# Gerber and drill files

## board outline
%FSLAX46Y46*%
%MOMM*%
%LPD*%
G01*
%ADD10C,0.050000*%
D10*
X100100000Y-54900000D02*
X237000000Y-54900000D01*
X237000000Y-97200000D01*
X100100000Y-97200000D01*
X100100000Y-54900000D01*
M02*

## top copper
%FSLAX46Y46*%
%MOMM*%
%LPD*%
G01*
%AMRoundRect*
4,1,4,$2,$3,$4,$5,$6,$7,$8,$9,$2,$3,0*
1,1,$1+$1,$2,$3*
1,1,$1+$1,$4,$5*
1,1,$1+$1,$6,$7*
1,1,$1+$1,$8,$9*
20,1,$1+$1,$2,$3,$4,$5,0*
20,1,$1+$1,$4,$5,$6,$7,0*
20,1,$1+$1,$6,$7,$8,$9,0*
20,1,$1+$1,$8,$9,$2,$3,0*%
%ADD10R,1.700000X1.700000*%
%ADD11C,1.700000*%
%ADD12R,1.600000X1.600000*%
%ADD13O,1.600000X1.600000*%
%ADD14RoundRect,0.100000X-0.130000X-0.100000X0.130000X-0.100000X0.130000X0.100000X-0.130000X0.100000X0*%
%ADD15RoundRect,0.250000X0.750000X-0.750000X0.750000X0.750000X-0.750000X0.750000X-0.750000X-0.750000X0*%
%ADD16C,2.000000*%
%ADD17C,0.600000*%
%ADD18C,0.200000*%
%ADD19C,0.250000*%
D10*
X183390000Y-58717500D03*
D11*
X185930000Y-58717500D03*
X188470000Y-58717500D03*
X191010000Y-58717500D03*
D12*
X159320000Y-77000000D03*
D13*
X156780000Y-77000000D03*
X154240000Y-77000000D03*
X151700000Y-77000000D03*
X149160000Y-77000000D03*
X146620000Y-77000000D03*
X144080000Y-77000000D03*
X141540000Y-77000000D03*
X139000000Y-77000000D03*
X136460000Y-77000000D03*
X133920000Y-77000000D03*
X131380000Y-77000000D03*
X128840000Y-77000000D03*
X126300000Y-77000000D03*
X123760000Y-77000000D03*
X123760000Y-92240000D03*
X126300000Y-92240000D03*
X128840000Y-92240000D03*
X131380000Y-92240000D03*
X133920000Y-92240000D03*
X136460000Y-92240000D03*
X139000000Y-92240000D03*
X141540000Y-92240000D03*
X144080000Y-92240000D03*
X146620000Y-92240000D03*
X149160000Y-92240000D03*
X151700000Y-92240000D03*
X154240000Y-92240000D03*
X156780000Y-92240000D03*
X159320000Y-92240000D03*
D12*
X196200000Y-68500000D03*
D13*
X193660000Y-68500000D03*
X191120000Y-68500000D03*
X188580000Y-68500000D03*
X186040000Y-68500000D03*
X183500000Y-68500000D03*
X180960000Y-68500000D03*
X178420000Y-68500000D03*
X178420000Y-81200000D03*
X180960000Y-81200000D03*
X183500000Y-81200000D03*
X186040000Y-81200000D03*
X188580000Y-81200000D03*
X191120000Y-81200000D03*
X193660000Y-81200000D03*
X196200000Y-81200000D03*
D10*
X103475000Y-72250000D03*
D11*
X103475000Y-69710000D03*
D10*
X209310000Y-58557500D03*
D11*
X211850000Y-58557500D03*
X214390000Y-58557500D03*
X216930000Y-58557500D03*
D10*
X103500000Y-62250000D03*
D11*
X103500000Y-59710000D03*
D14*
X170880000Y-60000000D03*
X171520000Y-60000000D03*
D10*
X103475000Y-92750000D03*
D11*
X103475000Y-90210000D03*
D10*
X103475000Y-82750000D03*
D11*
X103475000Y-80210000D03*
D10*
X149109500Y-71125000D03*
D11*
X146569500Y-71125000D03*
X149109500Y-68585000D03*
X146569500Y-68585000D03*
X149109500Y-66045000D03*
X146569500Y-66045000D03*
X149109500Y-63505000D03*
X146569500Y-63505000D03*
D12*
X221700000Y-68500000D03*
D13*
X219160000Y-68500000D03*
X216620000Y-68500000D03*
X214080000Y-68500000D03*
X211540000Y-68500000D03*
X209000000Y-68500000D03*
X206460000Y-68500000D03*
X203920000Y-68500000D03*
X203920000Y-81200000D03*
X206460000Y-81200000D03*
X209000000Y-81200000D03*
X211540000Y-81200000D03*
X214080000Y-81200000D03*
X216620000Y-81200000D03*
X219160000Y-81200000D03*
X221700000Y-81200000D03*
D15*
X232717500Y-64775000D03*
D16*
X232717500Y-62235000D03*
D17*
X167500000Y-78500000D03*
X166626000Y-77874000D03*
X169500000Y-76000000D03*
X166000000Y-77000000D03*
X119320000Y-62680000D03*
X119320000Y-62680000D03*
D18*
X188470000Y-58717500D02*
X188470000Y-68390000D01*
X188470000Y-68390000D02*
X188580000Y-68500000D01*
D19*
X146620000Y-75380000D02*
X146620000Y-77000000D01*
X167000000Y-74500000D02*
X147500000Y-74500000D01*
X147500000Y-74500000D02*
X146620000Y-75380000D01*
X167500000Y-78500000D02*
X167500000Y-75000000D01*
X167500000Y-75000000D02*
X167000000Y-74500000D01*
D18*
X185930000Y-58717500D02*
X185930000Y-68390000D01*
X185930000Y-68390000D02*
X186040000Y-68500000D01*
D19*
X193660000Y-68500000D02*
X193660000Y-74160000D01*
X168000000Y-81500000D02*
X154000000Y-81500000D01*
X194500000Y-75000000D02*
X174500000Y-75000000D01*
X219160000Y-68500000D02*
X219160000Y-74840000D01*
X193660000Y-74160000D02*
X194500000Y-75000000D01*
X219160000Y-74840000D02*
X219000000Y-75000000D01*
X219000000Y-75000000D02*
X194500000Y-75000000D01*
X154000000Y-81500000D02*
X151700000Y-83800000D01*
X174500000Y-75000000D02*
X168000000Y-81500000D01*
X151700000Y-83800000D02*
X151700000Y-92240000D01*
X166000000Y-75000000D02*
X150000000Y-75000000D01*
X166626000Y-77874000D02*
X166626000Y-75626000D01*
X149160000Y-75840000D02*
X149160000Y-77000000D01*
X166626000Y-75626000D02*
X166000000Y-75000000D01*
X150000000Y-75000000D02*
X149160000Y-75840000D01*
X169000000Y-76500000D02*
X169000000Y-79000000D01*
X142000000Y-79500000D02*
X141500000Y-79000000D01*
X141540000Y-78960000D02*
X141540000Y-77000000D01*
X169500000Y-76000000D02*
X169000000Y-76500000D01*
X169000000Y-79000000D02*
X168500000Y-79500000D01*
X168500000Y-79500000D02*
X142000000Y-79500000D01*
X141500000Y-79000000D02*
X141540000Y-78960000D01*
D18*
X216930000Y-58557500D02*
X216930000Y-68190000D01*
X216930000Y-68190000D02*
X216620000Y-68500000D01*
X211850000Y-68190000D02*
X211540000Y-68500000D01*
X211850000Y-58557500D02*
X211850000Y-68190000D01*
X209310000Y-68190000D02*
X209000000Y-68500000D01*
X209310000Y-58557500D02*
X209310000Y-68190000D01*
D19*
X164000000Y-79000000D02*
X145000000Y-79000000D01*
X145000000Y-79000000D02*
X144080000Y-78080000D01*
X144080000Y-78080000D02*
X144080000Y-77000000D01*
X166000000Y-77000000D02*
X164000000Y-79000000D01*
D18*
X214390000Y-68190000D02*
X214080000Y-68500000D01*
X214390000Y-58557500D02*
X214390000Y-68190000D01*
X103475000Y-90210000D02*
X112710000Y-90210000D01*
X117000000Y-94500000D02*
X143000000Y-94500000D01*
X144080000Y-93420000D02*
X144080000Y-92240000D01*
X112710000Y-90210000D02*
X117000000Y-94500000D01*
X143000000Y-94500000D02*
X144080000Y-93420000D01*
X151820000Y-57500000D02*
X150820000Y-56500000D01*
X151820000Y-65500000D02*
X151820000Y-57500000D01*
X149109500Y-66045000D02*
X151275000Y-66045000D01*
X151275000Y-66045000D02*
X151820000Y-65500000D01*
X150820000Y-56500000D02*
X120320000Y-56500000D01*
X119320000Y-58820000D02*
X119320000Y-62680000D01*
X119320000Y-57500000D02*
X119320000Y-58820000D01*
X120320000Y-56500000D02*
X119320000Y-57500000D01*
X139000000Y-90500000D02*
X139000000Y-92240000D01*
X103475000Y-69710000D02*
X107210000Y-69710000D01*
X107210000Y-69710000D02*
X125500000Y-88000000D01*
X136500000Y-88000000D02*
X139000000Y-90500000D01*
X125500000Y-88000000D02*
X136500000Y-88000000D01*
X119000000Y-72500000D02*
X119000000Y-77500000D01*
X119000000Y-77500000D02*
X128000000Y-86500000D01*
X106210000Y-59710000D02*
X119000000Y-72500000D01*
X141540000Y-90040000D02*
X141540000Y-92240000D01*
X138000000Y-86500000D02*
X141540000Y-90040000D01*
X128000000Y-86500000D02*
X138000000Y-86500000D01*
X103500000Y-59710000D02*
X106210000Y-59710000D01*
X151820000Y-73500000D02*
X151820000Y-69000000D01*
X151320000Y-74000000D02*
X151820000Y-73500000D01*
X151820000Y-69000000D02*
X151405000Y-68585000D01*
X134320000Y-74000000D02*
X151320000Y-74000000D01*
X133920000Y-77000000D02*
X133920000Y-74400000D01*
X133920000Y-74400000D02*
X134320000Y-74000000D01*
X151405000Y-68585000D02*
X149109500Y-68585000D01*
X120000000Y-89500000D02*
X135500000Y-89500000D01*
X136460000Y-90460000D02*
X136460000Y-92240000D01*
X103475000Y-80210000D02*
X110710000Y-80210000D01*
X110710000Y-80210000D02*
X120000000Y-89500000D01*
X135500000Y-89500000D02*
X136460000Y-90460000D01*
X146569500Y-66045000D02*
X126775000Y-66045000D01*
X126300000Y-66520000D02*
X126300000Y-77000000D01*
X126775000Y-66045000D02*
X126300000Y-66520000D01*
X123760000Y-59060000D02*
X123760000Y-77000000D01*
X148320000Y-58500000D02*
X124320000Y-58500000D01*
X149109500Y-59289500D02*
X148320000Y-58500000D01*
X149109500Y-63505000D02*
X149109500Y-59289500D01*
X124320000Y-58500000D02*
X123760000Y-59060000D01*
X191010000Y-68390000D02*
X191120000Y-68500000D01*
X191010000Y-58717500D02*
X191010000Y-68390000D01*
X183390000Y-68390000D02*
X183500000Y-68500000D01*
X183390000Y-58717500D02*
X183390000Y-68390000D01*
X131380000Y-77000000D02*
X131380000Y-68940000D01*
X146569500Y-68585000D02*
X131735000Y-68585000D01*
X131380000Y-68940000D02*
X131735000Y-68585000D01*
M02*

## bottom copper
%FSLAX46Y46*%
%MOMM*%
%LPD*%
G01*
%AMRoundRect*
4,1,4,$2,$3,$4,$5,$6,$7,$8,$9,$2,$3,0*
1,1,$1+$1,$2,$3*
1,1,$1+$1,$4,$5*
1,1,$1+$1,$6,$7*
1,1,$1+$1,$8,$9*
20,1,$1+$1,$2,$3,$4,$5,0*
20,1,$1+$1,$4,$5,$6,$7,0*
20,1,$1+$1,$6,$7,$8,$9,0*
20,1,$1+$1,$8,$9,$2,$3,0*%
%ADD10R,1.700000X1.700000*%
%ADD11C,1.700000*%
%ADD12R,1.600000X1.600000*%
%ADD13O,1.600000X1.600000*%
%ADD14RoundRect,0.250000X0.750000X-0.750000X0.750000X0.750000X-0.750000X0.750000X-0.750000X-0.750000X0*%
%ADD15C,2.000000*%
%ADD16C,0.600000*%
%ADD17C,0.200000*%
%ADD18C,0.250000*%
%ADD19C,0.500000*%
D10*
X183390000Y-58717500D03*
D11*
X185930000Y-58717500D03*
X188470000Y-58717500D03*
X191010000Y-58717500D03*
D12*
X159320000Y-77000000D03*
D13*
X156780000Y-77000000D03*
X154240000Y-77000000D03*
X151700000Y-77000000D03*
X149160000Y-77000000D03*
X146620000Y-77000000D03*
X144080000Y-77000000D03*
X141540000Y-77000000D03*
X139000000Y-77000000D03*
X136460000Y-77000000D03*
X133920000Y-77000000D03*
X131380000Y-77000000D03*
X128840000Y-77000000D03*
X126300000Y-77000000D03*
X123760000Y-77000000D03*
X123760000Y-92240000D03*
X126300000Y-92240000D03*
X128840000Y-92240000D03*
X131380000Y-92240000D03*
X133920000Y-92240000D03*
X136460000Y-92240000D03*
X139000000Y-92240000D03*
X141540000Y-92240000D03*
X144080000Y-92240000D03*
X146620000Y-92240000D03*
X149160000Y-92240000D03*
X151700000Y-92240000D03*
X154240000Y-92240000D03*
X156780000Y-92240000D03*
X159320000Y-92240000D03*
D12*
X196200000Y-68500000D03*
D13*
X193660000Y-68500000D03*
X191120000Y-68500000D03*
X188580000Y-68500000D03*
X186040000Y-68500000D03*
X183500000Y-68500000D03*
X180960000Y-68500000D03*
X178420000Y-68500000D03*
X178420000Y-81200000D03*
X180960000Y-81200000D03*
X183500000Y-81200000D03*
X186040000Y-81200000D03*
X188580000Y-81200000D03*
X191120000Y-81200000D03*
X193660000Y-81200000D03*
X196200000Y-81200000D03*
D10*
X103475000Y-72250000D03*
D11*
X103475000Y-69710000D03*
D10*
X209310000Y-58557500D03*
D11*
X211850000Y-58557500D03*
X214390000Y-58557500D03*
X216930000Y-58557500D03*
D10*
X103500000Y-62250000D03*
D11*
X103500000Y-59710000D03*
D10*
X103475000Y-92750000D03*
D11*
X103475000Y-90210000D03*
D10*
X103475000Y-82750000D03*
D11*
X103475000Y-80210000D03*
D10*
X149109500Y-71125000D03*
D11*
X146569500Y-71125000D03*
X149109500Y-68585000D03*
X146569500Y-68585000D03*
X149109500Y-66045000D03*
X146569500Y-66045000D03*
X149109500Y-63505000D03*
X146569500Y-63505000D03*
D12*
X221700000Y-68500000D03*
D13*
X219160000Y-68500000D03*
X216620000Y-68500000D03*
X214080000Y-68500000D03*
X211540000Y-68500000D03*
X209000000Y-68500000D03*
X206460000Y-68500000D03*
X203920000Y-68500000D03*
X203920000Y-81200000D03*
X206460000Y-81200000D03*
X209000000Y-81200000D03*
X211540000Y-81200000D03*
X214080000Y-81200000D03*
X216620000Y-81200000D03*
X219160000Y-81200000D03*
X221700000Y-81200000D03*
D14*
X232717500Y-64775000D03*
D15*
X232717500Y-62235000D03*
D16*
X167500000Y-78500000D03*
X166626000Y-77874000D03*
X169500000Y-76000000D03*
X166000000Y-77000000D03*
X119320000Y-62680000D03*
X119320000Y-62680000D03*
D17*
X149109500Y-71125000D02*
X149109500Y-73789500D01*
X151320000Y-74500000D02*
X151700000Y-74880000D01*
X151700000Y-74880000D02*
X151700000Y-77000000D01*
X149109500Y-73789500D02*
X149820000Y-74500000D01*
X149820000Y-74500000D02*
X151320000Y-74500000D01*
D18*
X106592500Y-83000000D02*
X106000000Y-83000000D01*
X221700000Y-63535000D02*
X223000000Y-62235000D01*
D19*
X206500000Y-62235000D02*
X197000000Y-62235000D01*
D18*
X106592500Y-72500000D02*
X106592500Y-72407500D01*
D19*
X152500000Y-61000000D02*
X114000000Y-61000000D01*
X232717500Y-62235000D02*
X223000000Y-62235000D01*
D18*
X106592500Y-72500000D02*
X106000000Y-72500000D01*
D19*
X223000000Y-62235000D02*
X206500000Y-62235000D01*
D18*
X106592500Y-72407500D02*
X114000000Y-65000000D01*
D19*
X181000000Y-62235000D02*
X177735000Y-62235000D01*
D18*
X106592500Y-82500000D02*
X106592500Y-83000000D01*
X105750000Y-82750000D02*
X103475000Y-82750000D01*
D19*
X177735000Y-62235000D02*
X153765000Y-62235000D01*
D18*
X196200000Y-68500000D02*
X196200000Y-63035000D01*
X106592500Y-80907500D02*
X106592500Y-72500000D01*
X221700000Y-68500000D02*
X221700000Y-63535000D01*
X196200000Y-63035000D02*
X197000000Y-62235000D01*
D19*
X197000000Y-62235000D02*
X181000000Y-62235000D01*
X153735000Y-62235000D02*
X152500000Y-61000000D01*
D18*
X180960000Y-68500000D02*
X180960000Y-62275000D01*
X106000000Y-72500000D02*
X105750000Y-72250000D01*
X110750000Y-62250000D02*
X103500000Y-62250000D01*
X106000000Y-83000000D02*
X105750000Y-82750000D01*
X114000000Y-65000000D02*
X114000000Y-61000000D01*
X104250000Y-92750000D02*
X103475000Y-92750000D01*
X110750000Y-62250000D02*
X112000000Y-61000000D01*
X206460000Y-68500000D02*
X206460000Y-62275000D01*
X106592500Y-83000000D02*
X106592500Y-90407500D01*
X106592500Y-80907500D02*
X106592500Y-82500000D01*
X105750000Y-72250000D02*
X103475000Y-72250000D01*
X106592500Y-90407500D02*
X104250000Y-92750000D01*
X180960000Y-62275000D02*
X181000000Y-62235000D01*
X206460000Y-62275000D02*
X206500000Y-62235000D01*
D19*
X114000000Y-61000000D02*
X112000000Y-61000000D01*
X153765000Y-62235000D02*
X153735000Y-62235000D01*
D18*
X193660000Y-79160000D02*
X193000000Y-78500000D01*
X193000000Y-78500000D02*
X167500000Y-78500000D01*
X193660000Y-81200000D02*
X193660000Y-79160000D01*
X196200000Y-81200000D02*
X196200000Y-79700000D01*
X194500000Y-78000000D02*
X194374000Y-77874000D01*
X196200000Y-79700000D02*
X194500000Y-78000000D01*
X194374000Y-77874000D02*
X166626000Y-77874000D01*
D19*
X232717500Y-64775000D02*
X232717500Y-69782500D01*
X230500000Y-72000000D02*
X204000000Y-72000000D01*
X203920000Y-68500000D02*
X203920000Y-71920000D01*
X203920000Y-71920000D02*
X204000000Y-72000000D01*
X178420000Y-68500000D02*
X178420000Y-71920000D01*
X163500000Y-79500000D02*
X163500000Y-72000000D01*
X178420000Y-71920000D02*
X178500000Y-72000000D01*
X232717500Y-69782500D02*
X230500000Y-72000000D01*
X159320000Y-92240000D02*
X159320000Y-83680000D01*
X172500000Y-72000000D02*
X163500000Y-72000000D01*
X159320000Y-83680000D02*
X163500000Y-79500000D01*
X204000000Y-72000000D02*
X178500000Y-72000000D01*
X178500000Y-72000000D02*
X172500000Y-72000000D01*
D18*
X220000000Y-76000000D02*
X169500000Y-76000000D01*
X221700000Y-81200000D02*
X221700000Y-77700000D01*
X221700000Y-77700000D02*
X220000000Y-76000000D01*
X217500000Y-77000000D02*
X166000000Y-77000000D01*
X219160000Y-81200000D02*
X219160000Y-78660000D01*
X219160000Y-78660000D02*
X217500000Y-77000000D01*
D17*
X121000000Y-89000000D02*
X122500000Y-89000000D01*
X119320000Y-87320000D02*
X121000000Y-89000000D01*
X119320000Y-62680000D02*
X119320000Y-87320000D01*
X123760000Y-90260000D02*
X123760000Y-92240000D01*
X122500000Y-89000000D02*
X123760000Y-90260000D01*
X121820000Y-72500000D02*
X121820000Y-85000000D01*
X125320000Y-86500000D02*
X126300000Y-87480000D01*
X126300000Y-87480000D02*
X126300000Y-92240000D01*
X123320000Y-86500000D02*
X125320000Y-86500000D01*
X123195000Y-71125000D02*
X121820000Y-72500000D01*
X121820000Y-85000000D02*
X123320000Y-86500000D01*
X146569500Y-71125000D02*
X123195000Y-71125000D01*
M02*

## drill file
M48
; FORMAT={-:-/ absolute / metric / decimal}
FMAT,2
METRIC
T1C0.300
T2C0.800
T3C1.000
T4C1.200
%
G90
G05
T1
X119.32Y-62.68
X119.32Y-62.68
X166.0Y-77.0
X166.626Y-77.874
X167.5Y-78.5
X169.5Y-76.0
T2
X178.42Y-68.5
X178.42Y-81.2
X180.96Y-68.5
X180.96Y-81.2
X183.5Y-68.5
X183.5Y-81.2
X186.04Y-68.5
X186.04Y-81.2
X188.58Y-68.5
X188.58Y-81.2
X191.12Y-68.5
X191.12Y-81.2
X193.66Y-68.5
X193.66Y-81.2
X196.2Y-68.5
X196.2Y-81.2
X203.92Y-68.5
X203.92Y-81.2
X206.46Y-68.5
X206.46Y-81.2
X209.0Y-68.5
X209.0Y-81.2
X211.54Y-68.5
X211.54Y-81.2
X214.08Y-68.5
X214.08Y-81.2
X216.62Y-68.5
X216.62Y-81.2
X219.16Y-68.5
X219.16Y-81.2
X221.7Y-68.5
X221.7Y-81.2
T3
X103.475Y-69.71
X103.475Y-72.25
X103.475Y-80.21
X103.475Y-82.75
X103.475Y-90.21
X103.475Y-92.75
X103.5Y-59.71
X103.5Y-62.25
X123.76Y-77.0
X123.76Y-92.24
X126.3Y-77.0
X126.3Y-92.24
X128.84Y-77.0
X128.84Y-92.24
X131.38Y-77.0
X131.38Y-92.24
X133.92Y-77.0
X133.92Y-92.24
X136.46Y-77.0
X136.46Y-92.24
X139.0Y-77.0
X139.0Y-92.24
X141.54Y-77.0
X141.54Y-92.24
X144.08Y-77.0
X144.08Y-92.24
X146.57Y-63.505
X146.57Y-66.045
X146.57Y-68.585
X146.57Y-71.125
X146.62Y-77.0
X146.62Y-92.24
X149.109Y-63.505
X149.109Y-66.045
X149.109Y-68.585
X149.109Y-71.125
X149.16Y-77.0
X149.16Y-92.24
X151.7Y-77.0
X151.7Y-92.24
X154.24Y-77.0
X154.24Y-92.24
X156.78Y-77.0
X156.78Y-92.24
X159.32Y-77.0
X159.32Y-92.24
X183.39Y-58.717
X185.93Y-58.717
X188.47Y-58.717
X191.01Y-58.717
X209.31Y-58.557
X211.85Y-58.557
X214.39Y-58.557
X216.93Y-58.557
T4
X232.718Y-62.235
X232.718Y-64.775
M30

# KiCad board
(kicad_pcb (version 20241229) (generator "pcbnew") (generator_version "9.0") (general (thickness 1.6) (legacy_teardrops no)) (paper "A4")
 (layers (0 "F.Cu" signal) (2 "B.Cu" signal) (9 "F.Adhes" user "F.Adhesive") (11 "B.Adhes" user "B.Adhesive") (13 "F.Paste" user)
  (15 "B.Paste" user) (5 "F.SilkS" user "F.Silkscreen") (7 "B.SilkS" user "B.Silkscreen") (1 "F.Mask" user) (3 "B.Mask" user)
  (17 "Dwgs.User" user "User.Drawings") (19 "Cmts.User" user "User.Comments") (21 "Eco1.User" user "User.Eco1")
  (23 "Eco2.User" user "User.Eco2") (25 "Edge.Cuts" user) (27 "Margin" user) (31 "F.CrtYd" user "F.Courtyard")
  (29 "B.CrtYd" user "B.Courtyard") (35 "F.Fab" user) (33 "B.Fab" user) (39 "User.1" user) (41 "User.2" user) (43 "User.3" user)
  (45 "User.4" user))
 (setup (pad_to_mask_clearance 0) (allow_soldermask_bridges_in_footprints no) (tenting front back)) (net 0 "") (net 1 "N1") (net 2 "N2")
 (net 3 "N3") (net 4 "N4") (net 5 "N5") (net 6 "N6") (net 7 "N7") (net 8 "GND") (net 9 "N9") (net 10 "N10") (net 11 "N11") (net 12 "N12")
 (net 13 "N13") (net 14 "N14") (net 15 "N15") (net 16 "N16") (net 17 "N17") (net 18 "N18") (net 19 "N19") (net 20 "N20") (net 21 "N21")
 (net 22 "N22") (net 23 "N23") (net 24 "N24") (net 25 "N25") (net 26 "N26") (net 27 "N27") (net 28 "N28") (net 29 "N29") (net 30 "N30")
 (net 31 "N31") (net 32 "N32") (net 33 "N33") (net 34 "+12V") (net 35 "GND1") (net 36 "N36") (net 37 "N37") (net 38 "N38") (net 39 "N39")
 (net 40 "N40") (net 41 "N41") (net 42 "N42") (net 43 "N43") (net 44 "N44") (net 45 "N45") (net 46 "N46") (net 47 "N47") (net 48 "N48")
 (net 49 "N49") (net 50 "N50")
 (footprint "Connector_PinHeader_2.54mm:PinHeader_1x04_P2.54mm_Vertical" (layer "F.Cu") (at 183.39 58.7175 90)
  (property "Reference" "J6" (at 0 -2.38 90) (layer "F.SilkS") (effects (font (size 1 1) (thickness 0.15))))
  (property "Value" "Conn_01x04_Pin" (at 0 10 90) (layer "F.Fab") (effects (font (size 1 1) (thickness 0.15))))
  (pad "1" thru_hole rect (at 0 0 90) (size 1.7 1.7) (drill 1) (layers "*.Cu" "*.Mask") (remove_unused_layers no) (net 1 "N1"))
  (pad "2" thru_hole circle (at 0 2.54 90) (size 1.7 1.7) (drill 1) (layers "*.Cu" "*.Mask") (remove_unused_layers no) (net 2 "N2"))
  (pad "3" thru_hole circle (at 0 5.08 90) (size 1.7 1.7) (drill 1) (layers "*.Cu" "*.Mask") (remove_unused_layers no) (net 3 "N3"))
  (pad "4" thru_hole circle (at 0 7.62 90) (size 1.7 1.7) (drill 1) (layers "*.Cu" "*.Mask") (remove_unused_layers no) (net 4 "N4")))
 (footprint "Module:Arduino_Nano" (layer "F.Cu") (at 159.32 77 -90)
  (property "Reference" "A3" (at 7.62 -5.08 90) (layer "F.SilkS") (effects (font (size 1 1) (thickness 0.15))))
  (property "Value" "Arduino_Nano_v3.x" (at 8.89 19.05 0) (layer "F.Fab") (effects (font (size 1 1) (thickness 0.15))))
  (pad "1" thru_hole rect (at 0 0 270) (size 1.6 1.6) (drill 1) (layers "*.Cu" "*.Mask") (remove_unused_layers no) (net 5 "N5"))
  (pad "2" thru_hole oval (at 0 2.54 270) (size 1.6 1.6) (drill 1) (layers "*.Cu" "*.Mask") (remove_unused_layers no) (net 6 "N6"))
  (pad "3" thru_hole oval (at 0 5.08 270) (size 1.6 1.6) (drill 1) (layers "*.Cu" "*.Mask") (remove_unused_layers no) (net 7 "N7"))
  (pad "4" thru_hole oval (at 0 7.62 270) (size 1.6 1.6) (drill 1) (layers "*.Cu" "*.Mask") (remove_unused_layers no) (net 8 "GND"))
  (pad "5" thru_hole oval (at 0 10.16 270) (size 1.6 1.6) (drill 1) (layers "*.Cu" "*.Mask") (remove_unused_layers no) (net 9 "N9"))
  (pad "6" thru_hole oval (at 0 12.7 270) (size 1.6 1.6) (drill 1) (layers "*.Cu" "*.Mask") (remove_unused_layers no) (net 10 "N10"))
  (pad "7" thru_hole oval (at 0 15.24 270) (size 1.6 1.6) (drill 1) (layers "*.Cu" "*.Mask") (remove_unused_layers no) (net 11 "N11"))
  (pad "8" thru_hole oval (at 0 17.78 270) (size 1.6 1.6) (drill 1) (layers "*.Cu" "*.Mask") (remove_unused_layers no) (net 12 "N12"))
  (pad "9" thru_hole oval (at 0 20.32 270) (size 1.6 1.6) (drill 1) (layers "*.Cu" "*.Mask") (remove_unused_layers no) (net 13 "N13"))
  (pad "10" thru_hole oval (at 0 22.86 270) (size 1.6 1.6) (drill 1) (layers "*.Cu" "*.Mask") (remove_unused_layers no) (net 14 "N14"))
  (pad "11" thru_hole oval (at 0 25.4 270) (size 1.6 1.6) (drill 1) (layers "*.Cu" "*.Mask") (remove_unused_layers no) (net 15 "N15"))
  (pad "12" thru_hole oval (at 0 27.94 270) (size 1.6 1.6) (drill 1) (layers "*.Cu" "*.Mask") (remove_unused_layers no) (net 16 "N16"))
  (pad "13" thru_hole oval (at 0 30.48 270) (size 1.6 1.6) (drill 1) (layers "*.Cu" "*.Mask") (remove_unused_layers no) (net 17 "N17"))
  (pad "14" thru_hole oval (at 0 33.02 270) (size 1.6 1.6) (drill 1) (layers "*.Cu" "*.Mask") (remove_unused_layers no) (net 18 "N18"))
  (pad "15" thru_hole oval (at 0 35.56 270) (size 1.6 1.6) (drill 1) (layers "*.Cu" "*.Mask") (remove_unused_layers no) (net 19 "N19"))
  (pad "16" thru_hole oval (at 15.24 35.56 270) (size 1.6 1.6) (drill 1) (layers "*.Cu" "*.Mask") (remove_unused_layers no) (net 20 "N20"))
  (pad "17" thru_hole oval (at 15.24 33.02 270) (size 1.6 1.6) (drill 1) (layers "*.Cu" "*.Mask") (remove_unused_layers no) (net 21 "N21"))
  (pad "18" thru_hole oval (at 15.24 30.48 270) (size 1.6 1.6) (drill 1) (layers "*.Cu" "*.Mask") (remove_unused_layers no) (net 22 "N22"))
  (pad "19" thru_hole oval (at 15.24 27.94 270) (size 1.6 1.6) (drill 1) (layers "*.Cu" "*.Mask") (remove_unused_layers no) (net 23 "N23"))
  (pad "20" thru_hole oval (at 15.24 25.4 270) (size 1.6 1.6) (drill 1) (layers "*.Cu" "*.Mask") (remove_unused_layers no) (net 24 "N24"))
  (pad "21" thru_hole oval (at 15.24 22.86 270) (size 1.6 1.6) (drill 1) (layers "*.Cu" "*.Mask") (remove_unused_layers no) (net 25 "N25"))
  (pad "22" thru_hole oval (at 15.24 20.32 270) (size 1.6 1.6) (drill 1) (layers "*.Cu" "*.Mask") (remove_unused_layers no) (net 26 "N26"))
  (pad "23" thru_hole oval (at 15.24 17.78 270) (size 1.6 1.6) (drill 1) (layers "*.Cu" "*.Mask") (remove_unused_layers no) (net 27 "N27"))
  (pad "24" thru_hole oval (at 15.24 15.24 270) (size 1.6 1.6) (drill 1) (layers "*.Cu" "*.Mask") (remove_unused_layers no) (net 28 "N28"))
  (pad "25" thru_hole oval (at 15.24 12.7 270) (size 1.6 1.6) (drill 1) (layers "*.Cu" "*.Mask") (remove_unused_layers no) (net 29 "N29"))
  (pad "26" thru_hole oval (at 15.24 10.16 270) (size 1.6 1.6) (drill 1) (layers "*.Cu" "*.Mask") (remove_unused_layers no) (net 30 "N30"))
  (pad "27" thru_hole oval (at 15.24 7.62 270) (size 1.6 1.6) (drill 1) (layers "*.Cu" "*.Mask") (remove_unused_layers no) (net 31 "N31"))
  (pad "28" thru_hole oval (at 15.24 5.08 270) (size 1.6 1.6) (drill 1) (layers "*.Cu" "*.Mask") (remove_unused_layers no) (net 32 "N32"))
  (pad "29" thru_hole oval (at 15.24 2.54 270) (size 1.6 1.6) (drill 1) (layers "*.Cu" "*.Mask") (remove_unused_layers no) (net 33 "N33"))
  (pad "30" thru_hole oval (at 15.24 0 270) (size 1.6 1.6) (drill 1) (layers "*.Cu" "*.Mask") (remove_unused_layers no) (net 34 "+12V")))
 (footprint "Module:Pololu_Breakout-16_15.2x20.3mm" (layer "F.Cu") (at 196.2 68.5 -90)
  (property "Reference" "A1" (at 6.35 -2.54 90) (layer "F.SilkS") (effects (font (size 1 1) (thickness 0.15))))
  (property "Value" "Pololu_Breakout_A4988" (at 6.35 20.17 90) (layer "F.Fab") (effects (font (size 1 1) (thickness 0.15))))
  (pad "1" thru_hole rect (at 0 0 270) (size 1.6 1.6) (drill 0.8) (layers "*.Cu" "*.Mask") (remove_unused_layers no) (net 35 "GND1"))
  (pad "2" thru_hole oval (at 0 2.54 270) (size 1.6 1.6) (drill 0.8) (layers "*.Cu" "*.Mask") (remove_unused_layers no) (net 31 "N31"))
  (pad "3" thru_hole oval (at 0 5.08 270) (size 1.6 1.6) (drill 0.8) (layers "*.Cu" "*.Mask") (remove_unused_layers no) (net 4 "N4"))
  (pad "4" thru_hole oval (at 0 7.62 270) (size 1.6 1.6) (drill 0.8) (layers "*.Cu" "*.Mask") (remove_unused_layers no) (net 3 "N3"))
  (pad "5" thru_hole oval (at 0 10.16 270) (size 1.6 1.6) (drill 0.8) (layers "*.Cu" "*.Mask") (remove_unused_layers no) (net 2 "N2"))
  (pad "6" thru_hole oval (at 0 12.7 270) (size 1.6 1.6) (drill 0.8) (layers "*.Cu" "*.Mask") (remove_unused_layers no) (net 1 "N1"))
  (pad "7" thru_hole oval (at 0 15.24 270) (size 1.6 1.6) (drill 0.8) (layers "*.Cu" "*.Mask") (remove_unused_layers no) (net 35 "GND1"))
  (pad "8" thru_hole oval (at 0 17.78 270) (size 1.6 1.6) (drill 0.8) (layers "*.Cu" "*.Mask") (remove_unused_layers no) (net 34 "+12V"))
  (pad "9" thru_hole oval (at 12.7 17.78 270) (size 1.6 1.6) (drill 0.8) (layers "*.Cu" "*.Mask") (remove_unused_layers no) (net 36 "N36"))
  (pad "10" thru_hole oval (at 12.7 15.24 270) (size 1.6 1.6) (drill 0.8) (layers "*.Cu" "*.Mask") (remove_unused_layers no) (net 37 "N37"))
  (pad "11" thru_hole oval (at 12.7 12.7 270) (size 1.6 1.6) (drill 0.8) (layers "*.Cu" "*.Mask") (remove_unused_layers no) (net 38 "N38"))
  (pad "12" thru_hole oval (at 12.7 10.16 270) (size 1.6 1.6) (drill 0.8) (layers "*.Cu" "*.Mask") (remove_unused_layers no) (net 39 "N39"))
  (pad "13" thru_hole oval (at 12.7 7.62 270) (size 1.6 1.6) (drill 0.8) (layers "*.Cu" "*.Mask") (remove_unused_layers no) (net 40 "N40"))
  (pad "14" thru_hole oval (at 12.7 5.08 270) (size 1.6 1.6) (drill 0.8) (layers "*.Cu" "*.Mask") (remove_unused_layers no) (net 40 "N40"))
  (pad "15" thru_hole oval (at 12.7 2.54 270) (size 1.6 1.6) (drill 0.8) (layers "*.Cu" "*.Mask") (remove_unused_layers no) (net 10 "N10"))
  (pad "16" thru_hole oval (at 12.7 0 270) (size 1.6 1.6) (drill 0.8) (layers "*.Cu" "*.Mask") (remove_unused_layers no) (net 9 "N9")))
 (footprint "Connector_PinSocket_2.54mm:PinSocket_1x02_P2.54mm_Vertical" (layer "F.Cu") (at 103.475 72.25 180)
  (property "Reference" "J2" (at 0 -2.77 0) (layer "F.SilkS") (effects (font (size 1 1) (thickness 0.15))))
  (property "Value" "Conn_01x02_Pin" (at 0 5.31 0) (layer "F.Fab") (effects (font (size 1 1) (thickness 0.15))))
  (pad "1" thru_hole rect (at 0 0 180) (size 1.7 1.7) (drill 1) (layers "*.Cu" "*.Mask") (remove_unused_layers no) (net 35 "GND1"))
  (pad "2" thru_hole circle (at 0 2.54 180) (size 1.7 1.7) (drill 1) (layers "*.Cu" "*.Mask") (remove_unused_layers no) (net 26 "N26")))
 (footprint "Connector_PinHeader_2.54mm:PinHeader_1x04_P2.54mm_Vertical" (layer "F.Cu") (at 209.31 58.5575 90)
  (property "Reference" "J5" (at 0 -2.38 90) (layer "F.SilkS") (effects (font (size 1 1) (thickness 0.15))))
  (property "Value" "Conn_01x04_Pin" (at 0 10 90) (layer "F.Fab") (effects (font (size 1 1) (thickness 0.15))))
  (pad "1" thru_hole rect (at 0 0 90) (size 1.7 1.7) (drill 1) (layers "*.Cu" "*.Mask") (remove_unused_layers no) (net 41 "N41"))
  (pad "2" thru_hole circle (at 0 2.54 90) (size 1.7 1.7) (drill 1) (layers "*.Cu" "*.Mask") (remove_unused_layers no) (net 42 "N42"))
  (pad "3" thru_hole circle (at 0 5.08 90) (size 1.7 1.7) (drill 1) (layers "*.Cu" "*.Mask") (remove_unused_layers no) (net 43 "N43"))
  (pad "4" thru_hole circle (at 0 7.62 90) (size 1.7 1.7) (drill 1) (layers "*.Cu" "*.Mask") (remove_unused_layers no) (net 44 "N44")))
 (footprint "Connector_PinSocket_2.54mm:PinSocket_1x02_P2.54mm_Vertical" (layer "F.Cu") (at 103.5 62.25 180)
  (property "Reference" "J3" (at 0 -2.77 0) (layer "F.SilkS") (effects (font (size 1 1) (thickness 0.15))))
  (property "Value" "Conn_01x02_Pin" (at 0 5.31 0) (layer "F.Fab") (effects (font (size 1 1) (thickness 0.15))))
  (pad "1" thru_hole rect (at 0 0 180) (size 1.7 1.7) (drill 1) (layers "*.Cu" "*.Mask") (remove_unused_layers no) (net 35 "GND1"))
  (pad "2" thru_hole circle (at 0 2.54 180) (size 1.7 1.7) (drill 1) (layers "*.Cu" "*.Mask") (remove_unused_layers no) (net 27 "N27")))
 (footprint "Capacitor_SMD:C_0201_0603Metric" (layer "F.Cu") (at 171.2 60)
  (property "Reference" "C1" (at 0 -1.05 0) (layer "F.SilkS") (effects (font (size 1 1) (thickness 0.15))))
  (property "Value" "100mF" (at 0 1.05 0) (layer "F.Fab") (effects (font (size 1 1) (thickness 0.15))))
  (pad "" smd roundrect (at -0.345 0) (size 0.318 0.36) (layers "F.Paste") (roundrect_rratio 0.25))
  (pad "" smd roundrect (at 0.345 0) (size 0.318 0.36) (layers "F.Paste") (roundrect_rratio 0.25))
  (pad "1" smd roundrect (at -0.32 0) (size 0.46 0.4) (layers "F.Cu" "F.Mask") (roundrect_rratio 0.25) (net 34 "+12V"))
  (pad "2" smd roundrect (at 0.32 0) (size 0.46 0.4) (layers "F.Cu" "F.Mask") (roundrect_rratio 0.25) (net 35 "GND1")))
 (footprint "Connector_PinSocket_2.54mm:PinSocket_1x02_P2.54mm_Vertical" (layer "F.Cu") (at 103.475 92.75 180)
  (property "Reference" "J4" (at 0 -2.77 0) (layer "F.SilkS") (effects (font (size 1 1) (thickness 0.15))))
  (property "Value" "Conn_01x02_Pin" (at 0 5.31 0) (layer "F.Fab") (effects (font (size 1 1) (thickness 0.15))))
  (pad "1" thru_hole rect (at 0 0 180) (size 1.7 1.7) (drill 1) (layers "*.Cu" "*.Mask") (remove_unused_layers no) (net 35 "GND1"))
  (pad "2" thru_hole circle (at 0 2.54 180) (size 1.7 1.7) (drill 1) (layers "*.Cu" "*.Mask") (remove_unused_layers no) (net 28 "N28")))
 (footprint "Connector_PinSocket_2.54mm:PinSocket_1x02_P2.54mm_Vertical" (layer "F.Cu") (at 103.475 82.75 180)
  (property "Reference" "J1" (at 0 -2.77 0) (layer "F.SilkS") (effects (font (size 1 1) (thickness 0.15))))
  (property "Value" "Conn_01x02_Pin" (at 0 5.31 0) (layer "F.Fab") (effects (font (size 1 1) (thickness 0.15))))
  (pad "1" thru_hole rect (at 0 0 180) (size 1.7 1.7) (drill 1) (layers "*.Cu" "*.Mask") (remove_unused_layers no) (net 35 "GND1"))
  (pad "2" thru_hole circle (at 0 2.54 180) (size 1.7 1.7) (drill 1) (layers "*.Cu" "*.Mask") (remove_unused_layers no) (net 25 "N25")))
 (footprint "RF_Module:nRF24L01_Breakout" (layer "F.Cu") (at 149.1095 71.125 180)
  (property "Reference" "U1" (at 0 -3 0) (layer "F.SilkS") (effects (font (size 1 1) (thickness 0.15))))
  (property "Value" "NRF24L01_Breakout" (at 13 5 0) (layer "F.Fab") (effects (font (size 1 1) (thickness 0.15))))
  (pad "1" thru_hole rect (at 0 0 180) (size 1.7 1.7) (drill 1) (layers "*.Cu" "*.Mask") (remove_unused_layers no) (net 8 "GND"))
  (pad "2" thru_hole circle (at 2.54 0 180) (size 1.7 1.7) (drill 1) (layers "*.Cu" "*.Mask") (remove_unused_layers no) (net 21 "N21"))
  (pad "3" thru_hole circle (at 0 2.54 180) (size 1.7 1.7) (drill 1) (layers "*.Cu" "*.Mask") (remove_unused_layers no) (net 15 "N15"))
  (pad "4" thru_hole circle (at 2.54 2.54 180) (size 1.7 1.7) (drill 1) (layers "*.Cu" "*.Mask") (remove_unused_layers no) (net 16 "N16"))
  (pad "5" thru_hole circle (at 0 5.08 180) (size 1.7 1.7) (drill 1) (layers "*.Cu" "*.Mask") (remove_unused_layers no) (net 20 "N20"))
  (pad "6" thru_hole circle (at 2.54 5.08 180) (size 1.7 1.7) (drill 1) (layers "*.Cu" "*.Mask") (remove_unused_layers no) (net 18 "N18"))
  (pad "7" thru_hole circle (at 0 7.62 180) (size 1.7 1.7) (drill 1) (layers "*.Cu" "*.Mask") (remove_unused_layers no) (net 19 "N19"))
  (pad "8" thru_hole circle (at 2.54 7.62 180) (size 1.7 1.7) (drill 1) (layers "*.Cu" "*.Mask") (remove_unused_layers no) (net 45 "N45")))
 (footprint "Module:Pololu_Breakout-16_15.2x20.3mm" (layer "F.Cu") (at 221.7 68.5 -90)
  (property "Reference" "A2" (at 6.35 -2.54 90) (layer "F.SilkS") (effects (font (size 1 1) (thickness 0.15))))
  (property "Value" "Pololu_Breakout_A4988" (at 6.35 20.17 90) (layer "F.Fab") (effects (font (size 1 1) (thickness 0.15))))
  (pad "1" thru_hole rect (at 0 0 270) (size 1.6 1.6) (drill 0.8) (layers "*.Cu" "*.Mask") (remove_unused_layers no) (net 35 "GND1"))
  (pad "2" thru_hole oval (at 0 2.54 270) (size 1.6 1.6) (drill 0.8) (layers "*.Cu" "*.Mask") (remove_unused_layers no) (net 31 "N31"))
  (pad "3" thru_hole oval (at 0 5.08 270) (size 1.6 1.6) (drill 0.8) (layers "*.Cu" "*.Mask") (remove_unused_layers no) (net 44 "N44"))
  (pad "4" thru_hole oval (at 0 7.62 270) (size 1.6 1.6) (drill 0.8) (layers "*.Cu" "*.Mask") (remove_unused_layers no) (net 43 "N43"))
  (pad "5" thru_hole oval (at 0 10.16 270) (size 1.6 1.6) (drill 0.8) (layers "*.Cu" "*.Mask") (remove_unused_layers no) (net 42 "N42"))
  (pad "6" thru_hole oval (at 0 12.7 270) (size 1.6 1.6) (drill 0.8) (layers "*.Cu" "*.Mask") (remove_unused_layers no) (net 41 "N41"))
  (pad "7" thru_hole oval (at 0 15.24 270) (size 1.6 1.6) (drill 0.8) (layers "*.Cu" "*.Mask") (remove_unused_layers no) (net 35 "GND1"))
  (pad "8" thru_hole oval (at 0 17.78 270) (size 1.6 1.6) (drill 0.8) (layers "*.Cu" "*.Mask") (remove_unused_layers no) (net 34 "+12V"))
  (pad "9" thru_hole oval (at 12.7 17.78 270) (size 1.6 1.6) (drill 0.8) (layers "*.Cu" "*.Mask") (remove_unused_layers no) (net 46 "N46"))
  (pad "10" thru_hole oval (at 12.7 15.24 270) (size 1.6 1.6) (drill 0.8) (layers "*.Cu" "*.Mask") (remove_unused_layers no) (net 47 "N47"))
  (pad "11" thru_hole oval (at 12.7 12.7 270) (size 1.6 1.6) (drill 0.8) (layers "*.Cu" "*.Mask") (remove_unused_layers no) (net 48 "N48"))
  (pad "12" thru_hole oval (at 12.7 10.16 270) (size 1.6 1.6) (drill 0.8) (layers "*.Cu" "*.Mask") (remove_unused_layers no) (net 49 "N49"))
  (pad "13" thru_hole oval (at 12.7 7.62 270) (size 1.6 1.6) (drill 0.8) (layers "*.Cu" "*.Mask") (remove_unused_layers no) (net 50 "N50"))
  (pad "14" thru_hole oval (at 12.7 5.08 270) (size 1.6 1.6) (drill 0.8) (layers "*.Cu" "*.Mask") (remove_unused_layers no) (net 50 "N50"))
  (pad "15" thru_hole oval (at 12.7 2.54 270) (size 1.6 1.6) (drill 0.8) (layers "*.Cu" "*.Mask") (remove_unused_layers no) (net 11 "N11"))
  (pad "16" thru_hole oval (at 12.7 0 270) (size 1.6 1.6) (drill 0.8) (layers "*.Cu" "*.Mask") (remove_unused_layers no) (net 12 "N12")))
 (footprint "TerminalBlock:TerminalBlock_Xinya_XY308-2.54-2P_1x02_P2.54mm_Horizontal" (layer "F.Cu") (at 232.7175 64.775 90)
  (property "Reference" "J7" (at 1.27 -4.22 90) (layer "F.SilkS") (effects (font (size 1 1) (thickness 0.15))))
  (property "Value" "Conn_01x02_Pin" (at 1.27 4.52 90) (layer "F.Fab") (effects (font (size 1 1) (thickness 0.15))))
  (pad "1" thru_hole roundrect (at 0 0 90) (size 2 2) (drill 1.2) (layers "*.Cu" "*.Mask") (remove_unused_layers no)
   (roundrect_rratio 0.125) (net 34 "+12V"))
  (pad "2" thru_hole circle (at 2.54 0 90) (size 2 2) (drill 1.2) (layers "*.Cu" "*.Mask") (remove_unused_layers no) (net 35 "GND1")))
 (gr_rect (start 100.1 54.9) (end 237 97.2) (stroke (width 0.05) (type default)) (fill no) (layer "Edge.Cuts"))
 (segment (start 149.1095 71.125) (end 149.1095 73.7895) (width 0.2) (layer "B.Cu") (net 8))
 (segment (start 151.32 74.5) (end 151.7 74.88) (width 0.2) (layer "B.Cu") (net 8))
 (segment (start 151.7 74.88) (end 151.7 77) (width 0.2) (layer "B.Cu") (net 8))
 (segment (start 149.1095 73.7895) (end 149.82 74.5) (width 0.2) (layer "B.Cu") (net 8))
 (segment (start 149.82 74.5) (end 151.32 74.5) (width 0.2) (layer "B.Cu") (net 8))
 (segment (start 106.5925 83) (end 106 83) (width 0.25) (layer "B.Cu") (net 35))
 (segment (start 221.7 63.535) (end 223 62.235) (width 0.25) (layer "B.Cu") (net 35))
 (segment (start 206.5 62.235) (end 197 62.235) (width 0.5) (layer "B.Cu") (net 35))
 (segment (start 106.5925 72.5) (end 106.5925 72.4075) (width 0.25) (layer "B.Cu") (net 35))
 (segment (start 152.5 61) (end 114 61) (width 0.5) (layer "B.Cu") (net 35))
 (segment (start 232.7175 62.235) (end 223 62.235) (width 0.5) (layer "B.Cu") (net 35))
 (segment (start 106.5925 72.5) (end 106 72.5) (width 0.25) (layer "B.Cu") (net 35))
 (segment (start 223 62.235) (end 206.5 62.235) (width 0.5) (layer "B.Cu") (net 35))
 (segment (start 106.5925 72.4075) (end 114 65) (width 0.25) (layer "B.Cu") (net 35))
 (segment (start 181 62.235) (end 177.735 62.235) (width 0.5) (layer "B.Cu") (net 35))
 (segment (start 106.5925 82.5) (end 106.5925 83) (width 0.25) (layer "B.Cu") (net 35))
 (segment (start 105.75 82.75) (end 103.475 82.75) (width 0.25) (layer "B.Cu") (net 35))
 (segment (start 177.735 62.235) (end 153.765 62.235) (width 0.5) (layer "B.Cu") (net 35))
 (segment (start 196.2 68.5) (end 196.2 63.035) (width 0.25) (layer "B.Cu") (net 35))
 (segment (start 106.5925 80.9075) (end 106.5925 72.5) (width 0.25) (layer "B.Cu") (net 35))
 (segment (start 221.7 68.5) (end 221.7 63.535) (width 0.25) (layer "B.Cu") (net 35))
 (segment (start 196.2 63.035) (end 197 62.235) (width 0.25) (layer "B.Cu") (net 35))
 (segment (start 197 62.235) (end 181 62.235) (width 0.5) (layer "B.Cu") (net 35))
 (segment (start 153.735 62.235) (end 152.5 61) (width 0.5) (layer "B.Cu") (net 35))
 (segment (start 180.96 68.5) (end 180.96 62.275) (width 0.25) (layer "B.Cu") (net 35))
 (segment (start 106 72.5) (end 105.75 72.25) (width 0.25) (layer "B.Cu") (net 35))
 (segment (start 110.75 62.25) (end 103.5 62.25) (width 0.25) (layer "B.Cu") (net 35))
 (segment (start 106 83) (end 105.75 82.75) (width 0.25) (layer "B.Cu") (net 35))
 (segment (start 114 65) (end 114 61) (width 0.25) (layer "B.Cu") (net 35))
 (segment (start 104.25 92.75) (end 103.475 92.75) (width 0.25) (layer "B.Cu") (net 35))
 (segment (start 110.75 62.25) (end 112 61) (width 0.25) (layer "B.Cu") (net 35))
 (segment (start 206.46 68.5) (end 206.46 62.275) (width 0.25) (layer "B.Cu") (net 35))
 (segment (start 106.5925 83) (end 106.5925 90.4075) (width 0.25) (layer "B.Cu") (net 35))
 (segment (start 106.5925 80.9075) (end 106.5925 82.5) (width 0.25) (layer "B.Cu") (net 35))
 (segment (start 105.75 72.25) (end 103.475 72.25) (width 0.25) (layer "B.Cu") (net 35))
 (segment (start 106.5925 90.4075) (end 104.25 92.75) (width 0.25) (layer "B.Cu") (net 35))
 (segment (start 180.96 62.275) (end 181 62.235) (width 0.25) (layer "B.Cu") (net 35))
 (segment (start 206.46 62.275) (end 206.5 62.235) (width 0.25) (layer "B.Cu") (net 35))
 (segment (start 114 61) (end 112 61) (width 0.5) (layer "B.Cu") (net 35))
 (segment (start 153.765 62.235) (end 153.735 62.235) (width 0.5) (layer "B.Cu") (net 35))
 (segment (start 188.47 58.7175) (end 188.47 68.39) (width 0.2) (layer "F.Cu") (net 3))
 (segment (start 188.47 68.39) (end 188.58 68.5) (width 0.2) (layer "F.Cu") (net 3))
 (segment (start 146.62 75.38) (end 146.62 77) (width 0.25) (layer "F.Cu") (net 10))
 (segment (start 167 74.5) (end 147.5 74.5) (width 0.25) (layer "F.Cu") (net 10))
 (segment (start 147.5 74.5) (end 146.62 75.38) (width 0.25) (layer "F.Cu") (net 10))
 (segment (start 167.5 78.5) (end 167.5 75) (width 0.25) (layer "F.Cu") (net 10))
 (segment (start 167.5 75) (end 167 74.5) (width 0.25) (layer "F.Cu") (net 10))
 (via (at 167.5 78.5) (size 0.6) (drill 0.3) (layers "F.Cu" "B.Cu") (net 10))
 (segment (start 193.66 79.16) (end 193 78.5) (width 0.25) (layer "B.Cu") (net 10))
 (segment (start 193 78.5) (end 167.5 78.5) (width 0.25) (layer "B.Cu") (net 10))
 (segment (start 193.66 81.2) (end 193.66 79.16) (width 0.25) (layer "B.Cu") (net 10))
 (segment (start 185.93 58.7175) (end 185.93 68.39) (width 0.2) (layer "F.Cu") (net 2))
 (segment (start 185.93 68.39) (end 186.04 68.5) (width 0.2) (layer "F.Cu") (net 2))
 (segment (start 193.66 68.5) (end 193.66 74.16) (width 0.25) (layer "F.Cu") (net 31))
 (segment (start 168 81.5) (end 154 81.5) (width 0.25) (layer "F.Cu") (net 31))
 (segment (start 194.5 75) (end 174.5 75) (width 0.25) (layer "F.Cu") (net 31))
 (segment (start 219.16 68.5) (end 219.16 74.84) (width 0.25) (layer "F.Cu") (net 31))
 (segment (start 193.66 74.16) (end 194.5 75) (width 0.25) (layer "F.Cu") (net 31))
 (segment (start 219.16 74.84) (end 219 75) (width 0.25) (layer "F.Cu") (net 31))
 (segment (start 219 75) (end 194.5 75) (width 0.25) (layer "F.Cu") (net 31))
 (segment (start 154 81.5) (end 151.7 83.8) (width 0.25) (layer "F.Cu") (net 31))
 (segment (start 174.5 75) (end 168 81.5) (width 0.25) (layer "F.Cu") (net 31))
 (segment (start 151.7 83.8) (end 151.7 92.24) (width 0.25) (layer "F.Cu") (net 31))
 (segment (start 166 75) (end 150 75) (width 0.25) (layer "F.Cu") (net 9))
 (segment (start 166.626 77.874) (end 166.626 75.626) (width 0.25) (layer "F.Cu") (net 9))
 (segment (start 149.16 75.84) (end 149.16 77) (width 0.25) (layer "F.Cu") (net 9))
 (segment (start 166.626 75.626) (end 166 75) (width 0.25) (layer "F.Cu") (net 9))
 (segment (start 150 75) (end 149.16 75.84) (width 0.25) (layer "F.Cu") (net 9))
 (via (at 166.626 77.874) (size 0.6) (drill 0.3) (layers "F.Cu" "B.Cu") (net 9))
 (segment (start 196.2 81.2) (end 196.2 79.7) (width 0.25) (layer "B.Cu") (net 9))
 (segment (start 194.5 78) (end 194.374 77.874) (width 0.25) (layer "B.Cu") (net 9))
 (segment (start 196.2 79.7) (end 194.5 78) (width 0.25) (layer "B.Cu") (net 9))
 (segment (start 194.374 77.874) (end 166.626 77.874) (width 0.25) (layer "B.Cu") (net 9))
 (segment (start 232.7175 64.775) (end 232.7175 69.7825) (width 0.5) (layer "B.Cu") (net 34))
 (segment (start 230.5 72) (end 204 72) (width 0.5) (layer "B.Cu") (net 34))
 (segment (start 203.92 68.5) (end 203.92 71.92) (width 0.5) (layer "B.Cu") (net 34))
 (segment (start 203.92 71.92) (end 204 72) (width 0.5) (layer "B.Cu") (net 34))
 (segment (start 178.42 68.5) (end 178.42 71.92) (width 0.5) (layer "B.Cu") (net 34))
 (segment (start 163.5 79.5) (end 163.5 72) (width 0.5) (layer "B.Cu") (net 34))
 (segment (start 178.42 71.92) (end 178.5 72) (width 0.5) (layer "B.Cu") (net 34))
 (segment (start 232.7175 69.7825) (end 230.5 72) (width 0.5) (layer "B.Cu") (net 34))
 (segment (start 159.32 92.24) (end 159.32 83.68) (width 0.5) (layer "B.Cu") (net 34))
 (segment (start 172.5 72) (end 163.5 72) (width 0.5) (layer "B.Cu") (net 34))
 (segment (start 159.32 83.68) (end 163.5 79.5) (width 0.5) (layer "B.Cu") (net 34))
 (segment (start 204 72) (end 178.5 72) (width 0.5) (layer "B.Cu") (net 34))
 (segment (start 178.5 72) (end 172.5 72) (width 0.5) (layer "B.Cu") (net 34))
 (segment (start 169 76.5) (end 169 79) (width 0.25) (layer "F.Cu") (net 12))
 (segment (start 142 79.5) (end 141.5 79) (width 0.25) (layer "F.Cu") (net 12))
 (segment (start 141.54 78.96) (end 141.54 77) (width 0.25) (layer "F.Cu") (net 12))
 (segment (start 169.5 76) (end 169 76.5) (width 0.25) (layer "F.Cu") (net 12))
 (segment (start 169 79) (end 168.5 79.5) (width 0.25) (layer "F.Cu") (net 12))
 (segment (start 168.5 79.5) (end 142 79.5) (width 0.25) (layer "F.Cu") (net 12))
 (segment (start 141.5 79) (end 141.54 78.96) (width 0.25) (layer "F.Cu") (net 12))
 (via (at 169.5 76) (size 0.6) (drill 0.3) (layers "F.Cu" "B.Cu") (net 12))
 (segment (start 220 76) (end 169.5 76) (width 0.25) (layer "B.Cu") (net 12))
 (segment (start 221.7 81.2) (end 221.7 77.7) (width 0.25) (layer "B.Cu") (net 12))
 (segment (start 221.7 77.7) (end 220 76) (width 0.25) (layer "B.Cu") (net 12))
 (segment (start 216.93 58.5575) (end 216.93 68.19) (width 0.2) (layer "F.Cu") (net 44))
 (segment (start 216.93 68.19) (end 216.62 68.5) (width 0.2) (layer "F.Cu") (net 44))
 (segment (start 211.85 68.19) (end 211.54 68.5) (width 0.2) (layer "F.Cu") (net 42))
 (segment (start 211.85 58.5575) (end 211.85 68.19) (width 0.2) (layer "F.Cu") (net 42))
 (segment (start 209.31 68.19) (end 209 68.5) (width 0.2) (layer "F.Cu") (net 41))
 (segment (start 209.31 58.5575) (end 209.31 68.19) (width 0.2) (layer "F.Cu") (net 41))
 (segment (start 164 79) (end 145 79) (width 0.25) (layer "F.Cu") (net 11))
 (segment (start 145 79) (end 144.08 78.08) (width 0.25) (layer "F.Cu") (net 11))
 (segment (start 144.08 78.08) (end 144.08 77) (width 0.25) (layer "F.Cu") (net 11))
 (segment (start 166 77) (end 164 79) (width 0.25) (layer "F.Cu") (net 11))
 (via (at 166 77) (size 0.6) (drill 0.3) (layers "F.Cu" "B.Cu") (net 11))
 (segment (start 217.5 77) (end 166 77) (width 0.25) (layer "B.Cu") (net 11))
 (segment (start 219.16 81.2) (end 219.16 78.66) (width 0.25) (layer "B.Cu") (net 11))
 (segment (start 219.16 78.66) (end 217.5 77) (width 0.25) (layer "B.Cu") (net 11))
 (segment (start 214.39 68.19) (end 214.08 68.5) (width 0.2) (layer "F.Cu") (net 43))
 (segment (start 214.39 58.5575) (end 214.39 68.19) (width 0.2) (layer "F.Cu") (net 43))
 (segment (start 103.475 90.21) (end 112.71 90.21) (width 0.2) (layer "F.Cu") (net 28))
 (segment (start 117 94.5) (end 143 94.5) (width 0.2) (layer "F.Cu") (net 28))
 (segment (start 144.08 93.42) (end 144.08 92.24) (width 0.2) (layer "F.Cu") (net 28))
 (segment (start 112.71 90.21) (end 117 94.5) (width 0.2) (layer "F.Cu") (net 28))
 (segment (start 143 94.5) (end 144.08 93.42) (width 0.2) (layer "F.Cu") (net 28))
 (segment (start 151.82 57.5) (end 150.82 56.5) (width 0.2) (layer "F.Cu") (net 20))
 (segment (start 151.82 65.5) (end 151.82 57.5) (width 0.2) (layer "F.Cu") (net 20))
 (segment (start 149.1095 66.045) (end 151.275 66.045) (width 0.2) (layer "F.Cu") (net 20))
 (segment (start 151.275 66.045) (end 151.82 65.5) (width 0.2) (layer "F.Cu") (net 20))
 (segment (start 150.82 56.5) (end 120.32 56.5) (width 0.2) (layer "F.Cu") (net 20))
 (segment (start 119.32 58.82) (end 119.32 62.68) (width 0.2) (layer "F.Cu") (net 20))
 (segment (start 119.32 57.5) (end 119.32 58.82) (width 0.2) (layer "F.Cu") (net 20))
 (segment (start 120.32 56.5) (end 119.32 57.5) (width 0.2) (layer "F.Cu") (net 20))
 (via (at 119.32 62.68) (size 0.6) (drill 0.3) (layers "F.Cu" "B.Cu") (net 20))
 (via (at 119.32 62.68) (size 0.6) (drill 0.3) (layers "F.Cu" "B.Cu") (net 20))
 (segment (start 121 89) (end 122.5 89) (width 0.2) (layer "B.Cu") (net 20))
 (segment (start 119.32 87.32) (end 121 89) (width 0.2) (layer "B.Cu") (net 20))
 (segment (start 119.32 62.68) (end 119.32 87.32) (width 0.2) (layer "B.Cu") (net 20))
 (segment (start 123.76 90.26) (end 123.76 92.24) (width 0.2) (layer "B.Cu") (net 20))
 (segment (start 122.5 89) (end 123.76 90.26) (width 0.2) (layer "B.Cu") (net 20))
 (segment (start 139 90.5) (end 139 92.24) (width 0.2) (layer "F.Cu") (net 26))
 (segment (start 103.475 69.71) (end 107.21 69.71) (width 0.2) (layer "F.Cu") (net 26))
 (segment (start 107.21 69.71) (end 125.5 88) (width 0.2) (layer "F.Cu") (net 26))
 (segment (start 136.5 88) (end 139 90.5) (width 0.2) (layer "F.Cu") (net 26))
 (segment (start 125.5 88) (end 136.5 88) (width 0.2) (layer "F.Cu") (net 26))
 (segment (start 119 72.5) (end 119 77.5) (width 0.2) (layer "F.Cu") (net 27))
 (segment (start 119 77.5) (end 128 86.5) (width 0.2) (layer "F.Cu") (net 27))
 (segment (start 106.21 59.71) (end 119 72.5) (width 0.2) (layer "F.Cu") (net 27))
 (segment (start 141.54 90.04) (end 141.54 92.24) (width 0.2) (layer "F.Cu") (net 27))
 (segment (start 138 86.5) (end 141.54 90.04) (width 0.2) (layer "F.Cu") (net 27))
 (segment (start 128 86.5) (end 138 86.5) (width 0.2) (layer "F.Cu") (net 27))
 (segment (start 103.5 59.71) (end 106.21 59.71) (width 0.2) (layer "F.Cu") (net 27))
 (segment (start 151.82 73.5) (end 151.82 69) (width 0.2) (layer "F.Cu") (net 15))
 (segment (start 151.32 74) (end 151.82 73.5) (width 0.2) (layer "F.Cu") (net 15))
 (segment (start 151.82 69) (end 151.405 68.585) (width 0.2) (layer "F.Cu") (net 15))
 (segment (start 134.32 74) (end 151.32 74) (width 0.2) (layer "F.Cu") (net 15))
 (segment (start 133.92 77) (end 133.92 74.4) (width 0.2) (layer "F.Cu") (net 15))
 (segment (start 133.92 74.4) (end 134.32 74) (width 0.2) (layer "F.Cu") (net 15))
 (segment (start 151.405 68.585) (end 149.1095 68.585) (width 0.2) (layer "F.Cu") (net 15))
 (segment (start 120 89.5) (end 135.5 89.5) (width 0.2) (layer "F.Cu") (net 25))
 (segment (start 136.46 90.46) (end 136.46 92.24) (width 0.2) (layer "F.Cu") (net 25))
 (segment (start 103.475 80.21) (end 110.71 80.21) (width 0.2) (layer "F.Cu") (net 25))
 (segment (start 110.71 80.21) (end 120 89.5) (width 0.2) (layer "F.Cu") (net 25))
 (segment (start 135.5 89.5) (end 136.46 90.46) (width 0.2) (layer "F.Cu") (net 25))
 (segment (start 146.5695 66.045) (end 126.775 66.045) (width 0.2) (layer "F.Cu") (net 18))
 (segment (start 126.3 66.52) (end 126.3 77) (width 0.2) (layer "F.Cu") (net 18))
 (segment (start 126.775 66.045) (end 126.3 66.52) (width 0.2) (layer "F.Cu") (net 18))
 (segment (start 123.76 59.06) (end 123.76 77) (width 0.2) (layer "F.Cu") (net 19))
 (segment (start 148.32 58.5) (end 124.32 58.5) (width 0.2) (layer "F.Cu") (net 19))
 (segment (start 149.1095 59.2895) (end 148.32 58.5) (width 0.2) (layer "F.Cu") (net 19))
 (segment (start 149.1095 63.505) (end 149.1095 59.2895) (width 0.2) (layer "F.Cu") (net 19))
 (segment (start 124.32 58.5) (end 123.76 59.06) (width 0.2) (layer "F.Cu") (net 19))
 (segment (start 191.01 68.39) (end 191.12 68.5) (width 0.2) (layer "F.Cu") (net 4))
 (segment (start 191.01 58.7175) (end 191.01 68.39) (width 0.2) (layer "F.Cu") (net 4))
 (segment (start 183.39 68.39) (end 183.5 68.5) (width 0.2) (layer "F.Cu") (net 1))
 (segment (start 183.39 58.7175) (end 183.39 68.39) (width 0.2) (layer "F.Cu") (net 1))
 (segment (start 121.82 72.5) (end 121.82 85) (width 0.2) (layer "B.Cu") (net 21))
 (segment (start 125.32 86.5) (end 126.3 87.48) (width 0.2) (layer "B.Cu") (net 21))
 (segment (start 126.3 87.48) (end 126.3 92.24) (width 0.2) (layer "B.Cu") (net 21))
 (segment (start 123.32 86.5) (end 125.32 86.5) (width 0.2) (layer "B.Cu") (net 21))
 (segment (start 123.195 71.125) (end 121.82 72.5) (width 0.2) (layer "B.Cu") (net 21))
 (segment (start 121.82 85) (end 123.32 86.5) (width 0.2) (layer "B.Cu") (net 21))
 (segment (start 146.5695 71.125) (end 123.195 71.125) (width 0.2) (layer "B.Cu") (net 21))
 (segment (start 131.38 77) (end 131.38 68.94) (width 0.2) (layer "F.Cu") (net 16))
 (segment (start 146.5695 68.585) (end 131.735 68.585) (width 0.2) (layer "F.Cu") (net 16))
 (segment (start 131.38 68.94) (end 131.735 68.585) (width 0.2) (layer "F.Cu") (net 16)))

